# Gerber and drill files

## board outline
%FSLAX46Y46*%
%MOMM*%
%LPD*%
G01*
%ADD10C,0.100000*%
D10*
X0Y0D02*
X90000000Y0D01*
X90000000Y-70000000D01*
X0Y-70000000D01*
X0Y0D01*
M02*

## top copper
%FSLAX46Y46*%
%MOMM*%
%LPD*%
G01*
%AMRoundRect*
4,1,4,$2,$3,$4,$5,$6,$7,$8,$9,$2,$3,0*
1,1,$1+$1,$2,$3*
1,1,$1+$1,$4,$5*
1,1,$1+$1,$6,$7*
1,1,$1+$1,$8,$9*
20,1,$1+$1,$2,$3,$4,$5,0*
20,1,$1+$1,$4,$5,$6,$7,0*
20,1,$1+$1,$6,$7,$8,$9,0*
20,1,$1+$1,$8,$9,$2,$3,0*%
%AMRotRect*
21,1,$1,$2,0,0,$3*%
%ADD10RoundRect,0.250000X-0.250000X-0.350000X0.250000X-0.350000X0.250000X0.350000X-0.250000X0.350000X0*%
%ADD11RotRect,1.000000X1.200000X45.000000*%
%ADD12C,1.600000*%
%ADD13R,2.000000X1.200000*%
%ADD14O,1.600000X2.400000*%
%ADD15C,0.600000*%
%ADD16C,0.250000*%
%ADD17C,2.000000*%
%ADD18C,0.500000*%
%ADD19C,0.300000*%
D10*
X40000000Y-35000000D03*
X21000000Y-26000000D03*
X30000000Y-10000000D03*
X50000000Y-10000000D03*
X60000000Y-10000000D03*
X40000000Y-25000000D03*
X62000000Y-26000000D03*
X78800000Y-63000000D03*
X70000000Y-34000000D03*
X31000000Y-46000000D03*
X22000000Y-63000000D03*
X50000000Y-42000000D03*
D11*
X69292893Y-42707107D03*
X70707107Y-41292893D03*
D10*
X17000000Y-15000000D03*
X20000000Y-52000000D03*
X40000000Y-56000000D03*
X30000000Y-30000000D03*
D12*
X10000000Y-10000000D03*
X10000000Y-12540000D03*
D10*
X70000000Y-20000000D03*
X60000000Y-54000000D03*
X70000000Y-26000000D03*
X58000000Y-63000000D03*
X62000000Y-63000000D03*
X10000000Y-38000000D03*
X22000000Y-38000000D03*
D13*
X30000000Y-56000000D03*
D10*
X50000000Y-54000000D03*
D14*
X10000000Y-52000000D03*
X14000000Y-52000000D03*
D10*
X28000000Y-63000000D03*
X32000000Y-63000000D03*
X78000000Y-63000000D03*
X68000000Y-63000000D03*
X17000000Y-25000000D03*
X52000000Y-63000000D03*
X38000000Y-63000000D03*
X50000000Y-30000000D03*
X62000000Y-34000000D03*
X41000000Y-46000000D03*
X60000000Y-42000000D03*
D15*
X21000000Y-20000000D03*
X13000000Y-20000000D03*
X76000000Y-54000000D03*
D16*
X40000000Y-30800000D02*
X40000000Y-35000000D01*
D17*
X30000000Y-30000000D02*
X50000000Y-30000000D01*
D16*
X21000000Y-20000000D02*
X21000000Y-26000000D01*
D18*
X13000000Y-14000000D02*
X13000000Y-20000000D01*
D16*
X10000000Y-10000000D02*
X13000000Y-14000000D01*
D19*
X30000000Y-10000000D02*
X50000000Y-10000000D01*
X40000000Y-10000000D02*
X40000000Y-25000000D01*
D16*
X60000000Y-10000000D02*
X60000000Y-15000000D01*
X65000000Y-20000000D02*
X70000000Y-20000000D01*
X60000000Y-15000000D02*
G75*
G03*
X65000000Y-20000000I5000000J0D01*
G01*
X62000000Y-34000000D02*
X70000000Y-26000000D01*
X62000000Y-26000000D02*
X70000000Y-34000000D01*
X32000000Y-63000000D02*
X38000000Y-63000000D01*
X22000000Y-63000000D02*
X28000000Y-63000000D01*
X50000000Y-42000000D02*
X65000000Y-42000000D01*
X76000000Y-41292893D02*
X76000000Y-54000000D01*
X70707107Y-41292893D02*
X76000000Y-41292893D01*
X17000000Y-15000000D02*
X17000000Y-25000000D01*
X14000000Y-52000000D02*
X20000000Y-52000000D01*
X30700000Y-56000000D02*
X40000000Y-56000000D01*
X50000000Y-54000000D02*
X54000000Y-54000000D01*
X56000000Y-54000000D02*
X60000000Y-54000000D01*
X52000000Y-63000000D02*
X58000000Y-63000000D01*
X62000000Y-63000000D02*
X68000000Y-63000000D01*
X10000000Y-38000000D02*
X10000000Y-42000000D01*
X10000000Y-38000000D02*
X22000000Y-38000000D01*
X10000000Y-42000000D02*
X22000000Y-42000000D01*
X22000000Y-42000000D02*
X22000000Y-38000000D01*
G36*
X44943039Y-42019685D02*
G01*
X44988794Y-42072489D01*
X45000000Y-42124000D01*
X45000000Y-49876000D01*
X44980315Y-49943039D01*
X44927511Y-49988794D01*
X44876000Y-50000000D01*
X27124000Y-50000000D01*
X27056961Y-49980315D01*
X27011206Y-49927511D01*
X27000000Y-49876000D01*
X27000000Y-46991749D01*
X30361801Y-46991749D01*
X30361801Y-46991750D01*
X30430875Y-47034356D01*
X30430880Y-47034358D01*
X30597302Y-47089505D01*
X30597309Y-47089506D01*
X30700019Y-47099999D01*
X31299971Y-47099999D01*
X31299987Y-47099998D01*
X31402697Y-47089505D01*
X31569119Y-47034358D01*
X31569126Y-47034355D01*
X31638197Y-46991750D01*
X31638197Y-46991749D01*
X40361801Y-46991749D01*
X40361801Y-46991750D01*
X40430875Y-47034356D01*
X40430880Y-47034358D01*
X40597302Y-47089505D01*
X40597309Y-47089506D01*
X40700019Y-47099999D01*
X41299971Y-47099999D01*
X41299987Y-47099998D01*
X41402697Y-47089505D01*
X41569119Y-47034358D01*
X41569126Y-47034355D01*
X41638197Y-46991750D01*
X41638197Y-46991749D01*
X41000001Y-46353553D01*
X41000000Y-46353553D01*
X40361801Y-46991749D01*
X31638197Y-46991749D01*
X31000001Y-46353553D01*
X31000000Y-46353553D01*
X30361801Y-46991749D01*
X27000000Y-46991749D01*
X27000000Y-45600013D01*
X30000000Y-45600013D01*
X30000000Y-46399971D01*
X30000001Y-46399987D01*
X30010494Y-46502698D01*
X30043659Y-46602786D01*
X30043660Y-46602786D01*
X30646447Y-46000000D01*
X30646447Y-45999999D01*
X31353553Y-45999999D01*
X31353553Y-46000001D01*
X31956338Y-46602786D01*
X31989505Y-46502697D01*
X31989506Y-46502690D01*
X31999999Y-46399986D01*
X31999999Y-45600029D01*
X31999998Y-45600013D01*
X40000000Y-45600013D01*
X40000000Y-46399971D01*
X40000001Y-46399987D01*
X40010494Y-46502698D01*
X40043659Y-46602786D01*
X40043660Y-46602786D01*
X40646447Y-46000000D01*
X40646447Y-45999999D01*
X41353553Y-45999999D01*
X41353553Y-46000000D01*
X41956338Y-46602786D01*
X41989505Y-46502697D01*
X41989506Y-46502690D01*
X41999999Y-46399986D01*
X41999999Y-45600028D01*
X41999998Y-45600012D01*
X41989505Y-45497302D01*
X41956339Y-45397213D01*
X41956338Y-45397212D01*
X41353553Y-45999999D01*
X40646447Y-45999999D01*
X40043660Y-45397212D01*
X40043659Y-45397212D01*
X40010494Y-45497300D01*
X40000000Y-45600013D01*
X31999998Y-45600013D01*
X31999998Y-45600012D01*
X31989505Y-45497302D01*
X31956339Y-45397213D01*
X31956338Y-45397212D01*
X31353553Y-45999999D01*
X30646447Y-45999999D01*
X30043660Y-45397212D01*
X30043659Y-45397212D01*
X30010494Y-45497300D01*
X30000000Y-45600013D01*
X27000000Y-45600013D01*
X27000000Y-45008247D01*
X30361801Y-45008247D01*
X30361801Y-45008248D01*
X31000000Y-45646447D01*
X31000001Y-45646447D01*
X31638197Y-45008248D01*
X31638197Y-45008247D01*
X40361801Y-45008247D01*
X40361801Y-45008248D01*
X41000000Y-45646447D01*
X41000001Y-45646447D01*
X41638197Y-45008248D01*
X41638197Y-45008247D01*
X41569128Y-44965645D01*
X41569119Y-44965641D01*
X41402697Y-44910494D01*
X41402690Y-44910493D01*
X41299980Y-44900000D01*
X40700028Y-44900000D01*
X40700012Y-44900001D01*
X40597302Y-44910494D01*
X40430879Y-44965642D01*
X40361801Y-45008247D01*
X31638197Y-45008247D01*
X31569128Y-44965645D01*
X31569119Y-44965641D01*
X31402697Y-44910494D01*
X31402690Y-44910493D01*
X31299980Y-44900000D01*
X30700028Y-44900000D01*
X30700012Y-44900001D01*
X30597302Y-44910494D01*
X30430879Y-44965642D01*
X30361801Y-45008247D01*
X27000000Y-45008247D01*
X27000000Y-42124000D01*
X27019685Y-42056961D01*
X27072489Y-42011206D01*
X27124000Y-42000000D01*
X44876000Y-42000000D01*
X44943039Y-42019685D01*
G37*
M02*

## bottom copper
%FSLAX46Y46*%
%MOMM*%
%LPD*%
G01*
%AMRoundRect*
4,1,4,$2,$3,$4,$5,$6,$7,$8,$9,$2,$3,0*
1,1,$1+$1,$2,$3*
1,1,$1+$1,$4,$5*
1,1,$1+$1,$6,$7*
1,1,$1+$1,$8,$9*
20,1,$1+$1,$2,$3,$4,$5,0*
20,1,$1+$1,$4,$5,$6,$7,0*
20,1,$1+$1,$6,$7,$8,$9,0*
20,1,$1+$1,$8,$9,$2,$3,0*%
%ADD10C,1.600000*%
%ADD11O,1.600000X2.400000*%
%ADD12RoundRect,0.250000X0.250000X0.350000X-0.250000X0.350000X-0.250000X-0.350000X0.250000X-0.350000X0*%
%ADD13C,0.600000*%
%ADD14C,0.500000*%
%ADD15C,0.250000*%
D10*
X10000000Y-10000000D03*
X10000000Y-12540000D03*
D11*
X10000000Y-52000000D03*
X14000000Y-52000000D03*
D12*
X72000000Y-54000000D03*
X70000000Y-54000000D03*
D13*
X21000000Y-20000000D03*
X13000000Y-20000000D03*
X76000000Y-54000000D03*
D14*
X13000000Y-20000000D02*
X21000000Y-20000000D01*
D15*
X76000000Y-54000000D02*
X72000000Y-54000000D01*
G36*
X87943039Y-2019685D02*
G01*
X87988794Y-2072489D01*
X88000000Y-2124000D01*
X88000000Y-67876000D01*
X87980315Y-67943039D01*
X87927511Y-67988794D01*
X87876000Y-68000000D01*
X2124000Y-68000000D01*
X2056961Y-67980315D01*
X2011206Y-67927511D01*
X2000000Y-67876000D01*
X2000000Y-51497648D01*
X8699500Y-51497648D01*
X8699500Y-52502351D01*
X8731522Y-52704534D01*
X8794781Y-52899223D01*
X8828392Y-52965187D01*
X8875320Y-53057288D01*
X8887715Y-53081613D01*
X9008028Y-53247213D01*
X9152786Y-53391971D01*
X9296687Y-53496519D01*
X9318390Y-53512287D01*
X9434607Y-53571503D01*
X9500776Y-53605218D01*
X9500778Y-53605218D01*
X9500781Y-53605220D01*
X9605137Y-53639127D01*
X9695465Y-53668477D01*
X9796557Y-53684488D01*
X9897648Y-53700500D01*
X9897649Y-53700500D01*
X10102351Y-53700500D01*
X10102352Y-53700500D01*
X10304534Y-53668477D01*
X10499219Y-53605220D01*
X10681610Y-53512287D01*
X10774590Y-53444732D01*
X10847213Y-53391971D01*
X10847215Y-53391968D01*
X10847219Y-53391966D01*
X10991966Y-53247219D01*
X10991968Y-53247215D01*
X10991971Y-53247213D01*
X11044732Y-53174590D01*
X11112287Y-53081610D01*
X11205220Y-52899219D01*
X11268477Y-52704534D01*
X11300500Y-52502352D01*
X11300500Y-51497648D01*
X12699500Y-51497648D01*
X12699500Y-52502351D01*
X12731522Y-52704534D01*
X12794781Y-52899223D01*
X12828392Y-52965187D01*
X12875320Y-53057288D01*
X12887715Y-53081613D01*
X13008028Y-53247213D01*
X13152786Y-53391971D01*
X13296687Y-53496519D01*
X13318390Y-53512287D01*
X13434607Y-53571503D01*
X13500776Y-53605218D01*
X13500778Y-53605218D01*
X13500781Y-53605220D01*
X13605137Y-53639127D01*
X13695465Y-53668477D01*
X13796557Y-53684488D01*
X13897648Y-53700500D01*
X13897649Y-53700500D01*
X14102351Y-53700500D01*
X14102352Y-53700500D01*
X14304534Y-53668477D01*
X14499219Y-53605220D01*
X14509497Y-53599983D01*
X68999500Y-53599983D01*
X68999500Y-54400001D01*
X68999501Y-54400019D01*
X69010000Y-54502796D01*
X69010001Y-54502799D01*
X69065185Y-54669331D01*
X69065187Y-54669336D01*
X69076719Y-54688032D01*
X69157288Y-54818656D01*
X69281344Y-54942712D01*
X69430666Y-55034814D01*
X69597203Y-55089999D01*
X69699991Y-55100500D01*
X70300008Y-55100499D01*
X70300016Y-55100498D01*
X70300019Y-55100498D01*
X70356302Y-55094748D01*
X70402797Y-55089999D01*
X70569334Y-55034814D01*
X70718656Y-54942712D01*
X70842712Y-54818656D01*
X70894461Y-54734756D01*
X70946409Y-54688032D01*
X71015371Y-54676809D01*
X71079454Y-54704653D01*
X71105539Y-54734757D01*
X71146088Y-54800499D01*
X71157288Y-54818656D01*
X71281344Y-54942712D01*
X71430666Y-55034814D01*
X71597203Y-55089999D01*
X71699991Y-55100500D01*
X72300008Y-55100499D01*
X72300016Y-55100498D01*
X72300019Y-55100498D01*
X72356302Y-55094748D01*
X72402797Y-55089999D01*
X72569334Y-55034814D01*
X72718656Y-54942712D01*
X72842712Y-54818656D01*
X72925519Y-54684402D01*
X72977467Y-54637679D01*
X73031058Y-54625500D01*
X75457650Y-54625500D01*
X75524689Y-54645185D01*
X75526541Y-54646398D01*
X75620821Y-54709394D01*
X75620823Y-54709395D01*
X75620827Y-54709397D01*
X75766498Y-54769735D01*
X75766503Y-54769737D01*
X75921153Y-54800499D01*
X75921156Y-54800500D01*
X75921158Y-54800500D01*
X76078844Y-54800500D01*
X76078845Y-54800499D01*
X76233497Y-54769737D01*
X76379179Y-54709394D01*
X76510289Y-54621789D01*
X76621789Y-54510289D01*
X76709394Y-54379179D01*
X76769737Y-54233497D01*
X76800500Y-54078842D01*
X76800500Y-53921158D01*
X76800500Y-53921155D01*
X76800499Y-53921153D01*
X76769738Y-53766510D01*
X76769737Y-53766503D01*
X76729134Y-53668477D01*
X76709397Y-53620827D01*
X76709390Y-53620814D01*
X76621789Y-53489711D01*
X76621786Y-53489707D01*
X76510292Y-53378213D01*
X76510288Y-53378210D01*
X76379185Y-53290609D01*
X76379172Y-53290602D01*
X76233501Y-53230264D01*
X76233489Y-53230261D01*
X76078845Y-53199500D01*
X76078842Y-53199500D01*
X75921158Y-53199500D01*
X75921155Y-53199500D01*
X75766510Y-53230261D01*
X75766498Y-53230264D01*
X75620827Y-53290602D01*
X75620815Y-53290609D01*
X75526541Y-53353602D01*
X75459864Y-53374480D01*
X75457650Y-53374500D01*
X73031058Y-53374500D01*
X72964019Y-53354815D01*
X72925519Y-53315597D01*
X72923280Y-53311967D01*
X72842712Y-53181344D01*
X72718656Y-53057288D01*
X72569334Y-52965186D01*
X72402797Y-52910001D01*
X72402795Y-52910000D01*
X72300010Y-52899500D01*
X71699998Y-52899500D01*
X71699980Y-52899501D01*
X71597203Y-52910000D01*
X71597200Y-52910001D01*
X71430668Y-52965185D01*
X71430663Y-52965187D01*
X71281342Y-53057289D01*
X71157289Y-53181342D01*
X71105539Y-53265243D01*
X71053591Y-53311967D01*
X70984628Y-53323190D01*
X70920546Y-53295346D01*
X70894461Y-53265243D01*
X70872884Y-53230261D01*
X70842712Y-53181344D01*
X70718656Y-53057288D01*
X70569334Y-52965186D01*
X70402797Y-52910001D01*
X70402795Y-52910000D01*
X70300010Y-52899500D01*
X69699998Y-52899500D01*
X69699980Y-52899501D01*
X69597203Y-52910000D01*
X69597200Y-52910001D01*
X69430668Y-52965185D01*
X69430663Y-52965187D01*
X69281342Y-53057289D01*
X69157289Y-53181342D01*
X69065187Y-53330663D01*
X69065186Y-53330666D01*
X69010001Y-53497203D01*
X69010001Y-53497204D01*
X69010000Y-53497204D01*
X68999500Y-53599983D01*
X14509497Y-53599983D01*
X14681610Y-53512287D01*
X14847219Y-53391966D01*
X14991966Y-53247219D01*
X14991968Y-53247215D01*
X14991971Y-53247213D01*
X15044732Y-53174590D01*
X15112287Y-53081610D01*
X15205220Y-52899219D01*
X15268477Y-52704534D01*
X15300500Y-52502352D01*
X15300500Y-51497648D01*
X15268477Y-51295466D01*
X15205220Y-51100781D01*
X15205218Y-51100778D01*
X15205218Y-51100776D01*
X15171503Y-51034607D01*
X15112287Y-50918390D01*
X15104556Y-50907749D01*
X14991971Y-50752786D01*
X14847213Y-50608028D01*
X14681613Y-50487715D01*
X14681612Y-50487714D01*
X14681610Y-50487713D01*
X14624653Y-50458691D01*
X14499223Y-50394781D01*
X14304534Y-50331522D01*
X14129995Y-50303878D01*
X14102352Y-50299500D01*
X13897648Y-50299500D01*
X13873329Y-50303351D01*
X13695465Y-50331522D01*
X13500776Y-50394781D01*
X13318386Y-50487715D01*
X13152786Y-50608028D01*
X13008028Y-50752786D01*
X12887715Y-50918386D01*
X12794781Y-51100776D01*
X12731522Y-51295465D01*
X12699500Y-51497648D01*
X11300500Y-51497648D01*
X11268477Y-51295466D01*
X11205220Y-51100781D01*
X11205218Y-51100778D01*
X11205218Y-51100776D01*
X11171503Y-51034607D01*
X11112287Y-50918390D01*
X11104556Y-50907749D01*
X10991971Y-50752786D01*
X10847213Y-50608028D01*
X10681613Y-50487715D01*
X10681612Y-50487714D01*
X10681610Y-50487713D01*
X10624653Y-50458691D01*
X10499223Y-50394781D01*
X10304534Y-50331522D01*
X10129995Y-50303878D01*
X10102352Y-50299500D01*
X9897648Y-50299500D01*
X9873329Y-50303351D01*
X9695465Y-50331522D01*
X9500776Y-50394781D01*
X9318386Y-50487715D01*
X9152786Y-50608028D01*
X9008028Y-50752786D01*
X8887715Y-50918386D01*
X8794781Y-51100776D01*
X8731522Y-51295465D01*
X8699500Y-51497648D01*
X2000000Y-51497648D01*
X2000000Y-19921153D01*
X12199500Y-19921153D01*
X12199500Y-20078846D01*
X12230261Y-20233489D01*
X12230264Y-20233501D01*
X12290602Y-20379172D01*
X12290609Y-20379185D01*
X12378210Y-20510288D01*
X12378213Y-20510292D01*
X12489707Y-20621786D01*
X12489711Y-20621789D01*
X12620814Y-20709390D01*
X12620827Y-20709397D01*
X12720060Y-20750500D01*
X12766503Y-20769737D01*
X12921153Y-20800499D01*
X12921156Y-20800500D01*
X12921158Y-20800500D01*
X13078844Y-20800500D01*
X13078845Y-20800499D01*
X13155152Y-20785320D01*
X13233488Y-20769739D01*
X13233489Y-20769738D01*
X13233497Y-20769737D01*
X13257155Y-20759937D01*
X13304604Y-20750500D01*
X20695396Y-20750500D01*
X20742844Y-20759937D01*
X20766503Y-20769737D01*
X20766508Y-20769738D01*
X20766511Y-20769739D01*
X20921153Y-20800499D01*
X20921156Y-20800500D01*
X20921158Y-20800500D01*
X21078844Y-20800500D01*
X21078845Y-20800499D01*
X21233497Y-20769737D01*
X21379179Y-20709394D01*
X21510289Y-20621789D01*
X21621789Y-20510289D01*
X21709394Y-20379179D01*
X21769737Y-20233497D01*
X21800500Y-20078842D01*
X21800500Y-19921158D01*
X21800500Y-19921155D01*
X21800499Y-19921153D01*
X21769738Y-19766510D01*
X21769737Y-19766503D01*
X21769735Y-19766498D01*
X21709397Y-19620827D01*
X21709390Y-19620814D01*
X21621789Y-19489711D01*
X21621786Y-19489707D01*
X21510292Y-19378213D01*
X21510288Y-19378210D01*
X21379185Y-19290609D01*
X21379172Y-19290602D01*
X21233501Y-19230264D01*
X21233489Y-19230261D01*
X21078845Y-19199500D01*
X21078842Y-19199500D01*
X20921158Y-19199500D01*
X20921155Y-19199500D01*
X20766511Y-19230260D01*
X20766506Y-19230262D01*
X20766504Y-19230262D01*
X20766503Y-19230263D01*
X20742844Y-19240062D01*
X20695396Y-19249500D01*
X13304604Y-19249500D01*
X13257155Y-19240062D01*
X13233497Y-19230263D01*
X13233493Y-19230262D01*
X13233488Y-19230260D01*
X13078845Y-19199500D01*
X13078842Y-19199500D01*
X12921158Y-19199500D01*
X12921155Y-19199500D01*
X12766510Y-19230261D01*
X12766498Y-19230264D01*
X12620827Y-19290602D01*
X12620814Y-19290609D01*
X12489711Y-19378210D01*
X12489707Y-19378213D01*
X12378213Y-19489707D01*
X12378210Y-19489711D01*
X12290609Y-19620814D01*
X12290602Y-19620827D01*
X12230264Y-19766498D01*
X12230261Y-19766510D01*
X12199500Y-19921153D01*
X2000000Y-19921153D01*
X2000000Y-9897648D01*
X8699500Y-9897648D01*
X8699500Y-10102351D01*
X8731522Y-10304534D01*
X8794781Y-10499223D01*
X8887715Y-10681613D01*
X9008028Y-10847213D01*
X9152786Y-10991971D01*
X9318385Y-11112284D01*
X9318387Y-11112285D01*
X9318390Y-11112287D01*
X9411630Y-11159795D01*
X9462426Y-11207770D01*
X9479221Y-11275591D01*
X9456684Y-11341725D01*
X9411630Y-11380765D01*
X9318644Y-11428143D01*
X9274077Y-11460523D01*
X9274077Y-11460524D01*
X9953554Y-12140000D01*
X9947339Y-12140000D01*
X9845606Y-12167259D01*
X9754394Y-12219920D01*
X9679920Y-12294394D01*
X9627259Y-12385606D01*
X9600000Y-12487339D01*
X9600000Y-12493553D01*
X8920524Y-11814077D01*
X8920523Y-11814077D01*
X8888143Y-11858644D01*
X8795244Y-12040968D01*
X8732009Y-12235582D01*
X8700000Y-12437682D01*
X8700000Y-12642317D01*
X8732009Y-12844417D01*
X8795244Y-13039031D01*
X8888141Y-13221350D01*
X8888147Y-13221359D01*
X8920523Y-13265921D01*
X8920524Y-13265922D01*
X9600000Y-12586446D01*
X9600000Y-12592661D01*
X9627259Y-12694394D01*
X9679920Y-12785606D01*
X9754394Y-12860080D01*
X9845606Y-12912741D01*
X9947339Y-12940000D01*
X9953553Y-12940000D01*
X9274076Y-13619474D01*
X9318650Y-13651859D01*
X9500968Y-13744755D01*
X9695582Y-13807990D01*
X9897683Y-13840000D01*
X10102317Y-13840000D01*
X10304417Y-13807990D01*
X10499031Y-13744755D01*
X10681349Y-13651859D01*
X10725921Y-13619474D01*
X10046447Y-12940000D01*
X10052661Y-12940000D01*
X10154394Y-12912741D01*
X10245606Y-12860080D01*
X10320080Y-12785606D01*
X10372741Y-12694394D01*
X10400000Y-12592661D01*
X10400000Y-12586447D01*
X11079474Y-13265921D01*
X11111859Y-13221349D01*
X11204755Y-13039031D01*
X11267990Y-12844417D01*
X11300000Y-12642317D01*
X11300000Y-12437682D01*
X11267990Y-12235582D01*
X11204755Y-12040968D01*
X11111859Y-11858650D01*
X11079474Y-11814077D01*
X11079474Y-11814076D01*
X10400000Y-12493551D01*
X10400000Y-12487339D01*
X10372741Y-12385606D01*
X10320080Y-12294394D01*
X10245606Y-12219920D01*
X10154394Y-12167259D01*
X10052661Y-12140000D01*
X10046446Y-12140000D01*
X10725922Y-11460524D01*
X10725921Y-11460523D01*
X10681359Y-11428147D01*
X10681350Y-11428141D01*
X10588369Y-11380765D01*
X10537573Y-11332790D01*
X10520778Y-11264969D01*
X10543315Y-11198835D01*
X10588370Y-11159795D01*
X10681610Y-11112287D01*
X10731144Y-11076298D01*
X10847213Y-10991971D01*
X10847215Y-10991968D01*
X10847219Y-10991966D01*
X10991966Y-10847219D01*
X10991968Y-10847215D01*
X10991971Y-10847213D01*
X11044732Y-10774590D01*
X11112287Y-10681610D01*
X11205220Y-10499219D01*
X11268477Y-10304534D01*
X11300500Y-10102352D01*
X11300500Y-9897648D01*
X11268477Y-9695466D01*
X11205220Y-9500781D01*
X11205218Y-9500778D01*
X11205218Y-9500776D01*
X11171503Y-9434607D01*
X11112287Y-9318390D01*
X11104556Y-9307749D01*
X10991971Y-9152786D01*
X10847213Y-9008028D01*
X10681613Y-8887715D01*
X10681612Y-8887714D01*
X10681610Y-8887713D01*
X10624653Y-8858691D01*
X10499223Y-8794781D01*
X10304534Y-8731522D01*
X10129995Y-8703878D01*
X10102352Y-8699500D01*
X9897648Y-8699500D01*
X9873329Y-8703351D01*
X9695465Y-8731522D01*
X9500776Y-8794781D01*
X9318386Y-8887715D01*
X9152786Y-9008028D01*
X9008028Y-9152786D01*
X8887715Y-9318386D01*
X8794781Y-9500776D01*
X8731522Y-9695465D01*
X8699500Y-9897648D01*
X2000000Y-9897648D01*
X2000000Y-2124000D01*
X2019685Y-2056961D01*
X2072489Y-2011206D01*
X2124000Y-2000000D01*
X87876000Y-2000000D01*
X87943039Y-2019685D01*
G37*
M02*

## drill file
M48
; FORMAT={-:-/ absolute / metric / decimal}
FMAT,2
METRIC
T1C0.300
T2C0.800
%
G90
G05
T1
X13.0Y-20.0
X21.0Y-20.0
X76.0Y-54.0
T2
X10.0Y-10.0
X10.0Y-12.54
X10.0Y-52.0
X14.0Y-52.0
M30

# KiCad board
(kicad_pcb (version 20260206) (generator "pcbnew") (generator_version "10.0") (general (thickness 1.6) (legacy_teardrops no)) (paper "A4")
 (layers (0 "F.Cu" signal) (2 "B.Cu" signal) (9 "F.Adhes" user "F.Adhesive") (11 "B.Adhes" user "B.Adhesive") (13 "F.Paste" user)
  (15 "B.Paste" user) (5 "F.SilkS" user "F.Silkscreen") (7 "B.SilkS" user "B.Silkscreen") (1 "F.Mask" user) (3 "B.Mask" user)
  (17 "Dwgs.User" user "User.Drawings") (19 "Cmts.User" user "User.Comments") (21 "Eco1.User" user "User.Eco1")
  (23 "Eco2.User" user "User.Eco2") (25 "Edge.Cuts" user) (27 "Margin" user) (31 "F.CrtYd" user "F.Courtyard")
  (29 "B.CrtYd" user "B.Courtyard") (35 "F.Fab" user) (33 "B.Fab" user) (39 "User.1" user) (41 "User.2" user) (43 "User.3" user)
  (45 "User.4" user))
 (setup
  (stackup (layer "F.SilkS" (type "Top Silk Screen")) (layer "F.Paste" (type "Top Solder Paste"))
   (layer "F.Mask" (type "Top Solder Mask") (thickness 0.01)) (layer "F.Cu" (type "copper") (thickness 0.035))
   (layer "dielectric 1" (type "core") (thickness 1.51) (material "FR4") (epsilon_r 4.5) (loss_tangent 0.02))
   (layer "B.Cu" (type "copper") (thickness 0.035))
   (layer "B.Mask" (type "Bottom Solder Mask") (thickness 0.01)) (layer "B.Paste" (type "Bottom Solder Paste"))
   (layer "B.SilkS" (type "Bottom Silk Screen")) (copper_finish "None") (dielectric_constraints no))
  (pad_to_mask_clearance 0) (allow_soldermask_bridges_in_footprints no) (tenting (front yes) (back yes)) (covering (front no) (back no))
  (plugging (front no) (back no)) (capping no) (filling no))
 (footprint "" (layer "F.Cu") (at 40 35)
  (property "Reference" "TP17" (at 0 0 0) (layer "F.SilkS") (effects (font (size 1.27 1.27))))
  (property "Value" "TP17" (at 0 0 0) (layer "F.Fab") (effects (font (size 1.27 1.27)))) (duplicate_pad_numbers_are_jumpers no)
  (pad "1" smd roundrect (at 0 0) (size 1 1.2) (layers "F.Cu" "F.Mask" "F.Paste") (roundrect_rratio 0.25) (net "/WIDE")
   (thermal_bridge_angle 45)))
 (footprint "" (layer "F.Cu") (at 21 26)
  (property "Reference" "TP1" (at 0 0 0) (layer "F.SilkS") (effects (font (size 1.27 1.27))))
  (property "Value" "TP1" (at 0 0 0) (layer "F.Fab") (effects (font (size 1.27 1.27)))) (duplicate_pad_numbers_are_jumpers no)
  (pad "1" smd roundrect (at 0 0) (size 1 1.2) (layers "F.Cu" "F.Mask" "F.Paste") (roundrect_rratio 0.25) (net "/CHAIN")
   (thermal_bridge_angle 45)))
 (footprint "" (layer "F.Cu") (at 30 10)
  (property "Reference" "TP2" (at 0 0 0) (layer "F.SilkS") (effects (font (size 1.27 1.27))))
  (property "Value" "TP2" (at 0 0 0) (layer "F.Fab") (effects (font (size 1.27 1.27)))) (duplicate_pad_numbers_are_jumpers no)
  (pad "1" smd roundrect (at 0 0) (size 1 1.2) (layers "F.Cu" "F.Mask" "F.Paste") (roundrect_rratio 0.25) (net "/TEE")
   (thermal_bridge_angle 45)))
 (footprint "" (layer "F.Cu") (at 50 10)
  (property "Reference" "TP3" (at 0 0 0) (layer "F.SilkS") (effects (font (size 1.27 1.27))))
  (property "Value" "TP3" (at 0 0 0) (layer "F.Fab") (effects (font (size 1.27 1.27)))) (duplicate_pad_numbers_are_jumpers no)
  (pad "1" smd roundrect (at 0 0) (size 1 1.2) (layers "F.Cu" "F.Mask" "F.Paste") (roundrect_rratio 0.25) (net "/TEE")
   (thermal_bridge_angle 45)))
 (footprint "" (layer "F.Cu") (at 60 10)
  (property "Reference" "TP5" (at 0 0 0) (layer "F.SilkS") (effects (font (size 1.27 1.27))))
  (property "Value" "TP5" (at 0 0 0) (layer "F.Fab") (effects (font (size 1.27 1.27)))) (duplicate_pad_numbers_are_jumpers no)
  (pad "1" smd roundrect (at 0 0) (size 1 1.2) (layers "F.Cu" "F.Mask" "F.Paste") (roundrect_rratio 0.25) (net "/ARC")
   (thermal_bridge_angle 45)))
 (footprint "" (layer "F.Cu") (at 40 25)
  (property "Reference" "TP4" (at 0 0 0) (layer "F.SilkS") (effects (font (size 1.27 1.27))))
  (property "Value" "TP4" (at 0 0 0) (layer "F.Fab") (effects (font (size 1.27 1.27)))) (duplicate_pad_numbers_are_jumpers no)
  (pad "1" smd roundrect (at 0 0) (size 1 1.2) (layers "F.Cu" "F.Mask" "F.Paste") (roundrect_rratio 0.25) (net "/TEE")
   (thermal_bridge_angle 45)))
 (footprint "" (layer "F.Cu") (at 62 26)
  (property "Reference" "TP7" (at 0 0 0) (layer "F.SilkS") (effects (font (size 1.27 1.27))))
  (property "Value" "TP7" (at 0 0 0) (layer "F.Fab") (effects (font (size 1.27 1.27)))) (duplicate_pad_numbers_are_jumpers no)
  (pad "1" smd roundrect (at 0 0) (size 1 1.2) (layers "F.Cu" "F.Mask" "F.Paste") (roundrect_rratio 0.25) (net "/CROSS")
   (thermal_bridge_angle 45)))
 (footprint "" (layer "F.Cu") (at 78.8 63)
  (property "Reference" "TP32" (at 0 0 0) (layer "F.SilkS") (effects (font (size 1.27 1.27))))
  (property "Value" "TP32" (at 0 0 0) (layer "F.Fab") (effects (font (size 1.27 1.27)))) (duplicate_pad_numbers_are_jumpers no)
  (pad "1" smd roundrect (at 0 0) (size 1 1.2) (layers "F.Cu" "F.Mask" "F.Paste") (roundrect_rratio 0.25) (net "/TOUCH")
   (thermal_bridge_angle 45)))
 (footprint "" (layer "F.Cu") (at 70 34)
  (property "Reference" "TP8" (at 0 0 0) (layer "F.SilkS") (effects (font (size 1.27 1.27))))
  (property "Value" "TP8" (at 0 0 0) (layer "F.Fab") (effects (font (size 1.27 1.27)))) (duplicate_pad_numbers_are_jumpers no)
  (pad "1" smd roundrect (at 0 0) (size 1 1.2) (layers "F.Cu" "F.Mask" "F.Paste") (roundrect_rratio 0.25) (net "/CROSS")
   (thermal_bridge_angle 45)))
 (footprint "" (layer "F.Cu") (at 31 46)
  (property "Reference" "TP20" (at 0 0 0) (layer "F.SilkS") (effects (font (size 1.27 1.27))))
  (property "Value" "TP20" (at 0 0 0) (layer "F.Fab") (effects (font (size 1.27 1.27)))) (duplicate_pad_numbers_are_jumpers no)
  (pad "1" smd roundrect (at 0 0) (size 1 1.2) (layers "F.Cu" "F.Mask" "F.Paste") (roundrect_rratio 0.25) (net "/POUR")
   (thermal_bridge_angle 45)))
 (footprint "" (layer "F.Cu") (at 22 63)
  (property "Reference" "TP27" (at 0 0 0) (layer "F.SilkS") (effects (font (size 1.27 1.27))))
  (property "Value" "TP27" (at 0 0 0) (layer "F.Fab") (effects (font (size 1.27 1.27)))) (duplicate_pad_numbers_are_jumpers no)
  (pad "1" smd roundrect (at 0 0) (size 1 1.2) (layers "F.Cu" "F.Mask" "F.Paste") (roundrect_rratio 0.25) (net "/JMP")
   (thermal_bridge_angle 45)))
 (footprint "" (layer "F.Cu") (at 50 42)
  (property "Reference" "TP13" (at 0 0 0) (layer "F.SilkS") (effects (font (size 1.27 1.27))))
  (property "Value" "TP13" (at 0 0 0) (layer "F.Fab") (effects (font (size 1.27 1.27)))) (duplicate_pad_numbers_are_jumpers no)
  (pad "1" smd roundrect (at 0 0) (size 1 1.2) (layers "F.Cu" "F.Mask" "F.Paste") (roundrect_rratio 0.25) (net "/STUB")
   (thermal_bridge_angle 45)))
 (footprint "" (layer "F.Cu") (at 70 42 45)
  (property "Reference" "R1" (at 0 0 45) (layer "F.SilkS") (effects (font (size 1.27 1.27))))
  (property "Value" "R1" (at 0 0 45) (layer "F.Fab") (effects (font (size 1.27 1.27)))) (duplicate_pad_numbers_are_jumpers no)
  (pad "1" smd rect (at -1 0 45) (size 1 1.2) (layers "F.Cu" "F.Mask" "F.Paste") (thermal_bridge_angle 45))
  (pad "2" smd rect (at 1 0 45) (size 1 1.2) (layers "F.Cu" "F.Mask" "F.Paste") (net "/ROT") (thermal_bridge_angle 45)))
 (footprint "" (layer "F.Cu") (at 17 15)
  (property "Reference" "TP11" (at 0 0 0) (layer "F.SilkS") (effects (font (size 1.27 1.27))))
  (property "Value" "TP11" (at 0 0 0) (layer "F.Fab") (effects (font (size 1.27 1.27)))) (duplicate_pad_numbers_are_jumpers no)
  (pad "1" smd roundrect (at 0 0) (size 1 1.2) (layers "F.Cu" "F.Mask" "F.Paste") (roundrect_rratio 0.25) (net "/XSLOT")
   (thermal_bridge_angle 45)))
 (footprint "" (layer "F.Cu") (at 20 52)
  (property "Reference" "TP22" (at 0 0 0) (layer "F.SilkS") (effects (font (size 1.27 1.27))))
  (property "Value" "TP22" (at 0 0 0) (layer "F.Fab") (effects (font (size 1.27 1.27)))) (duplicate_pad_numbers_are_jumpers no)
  (pad "1" smd roundrect (at 0 0) (size 1 1.2) (layers "F.Cu" "F.Mask" "F.Paste") (roundrect_rratio 0.25) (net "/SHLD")
   (thermal_bridge_angle 45)))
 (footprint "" (layer "F.Cu") (at 40 56)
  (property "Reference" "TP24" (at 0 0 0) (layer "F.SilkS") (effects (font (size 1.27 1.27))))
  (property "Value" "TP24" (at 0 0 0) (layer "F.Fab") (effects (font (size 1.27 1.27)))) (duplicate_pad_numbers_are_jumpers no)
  (pad "1" smd roundrect (at 0 0) (size 1 1.2) (layers "F.Cu" "F.Mask" "F.Paste") (roundrect_rratio 0.25) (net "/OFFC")
   (thermal_bridge_angle 45)))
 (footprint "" (layer "F.Cu") (at 30 30)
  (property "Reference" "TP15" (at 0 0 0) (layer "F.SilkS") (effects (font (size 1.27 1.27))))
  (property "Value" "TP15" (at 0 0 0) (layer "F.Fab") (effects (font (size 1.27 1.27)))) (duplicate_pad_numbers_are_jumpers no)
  (pad "1" smd roundrect (at 0 0) (size 1 1.2) (layers "F.Cu" "F.Mask" "F.Paste") (roundrect_rratio 0.25) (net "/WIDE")
   (thermal_bridge_angle 45)))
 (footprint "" (layer "F.Cu") (at 10 10)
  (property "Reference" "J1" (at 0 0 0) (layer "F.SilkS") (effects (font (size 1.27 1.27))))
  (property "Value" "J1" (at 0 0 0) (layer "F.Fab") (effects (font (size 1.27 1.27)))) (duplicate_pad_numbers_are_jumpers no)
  (pad "1" thru_hole circle (at 0 0) (size 1.6 1.6) (drill 0.8) (layers "*.Cu" "*.Mask") (remove_unused_layers no) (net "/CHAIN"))
  (pad "2" thru_hole circle (at 0 2.54) (size 1.6 1.6) (drill 0.8) (layers "*.Cu" "*.Mask") (remove_unused_layers no) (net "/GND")))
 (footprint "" (layer "F.Cu") (at 70 20)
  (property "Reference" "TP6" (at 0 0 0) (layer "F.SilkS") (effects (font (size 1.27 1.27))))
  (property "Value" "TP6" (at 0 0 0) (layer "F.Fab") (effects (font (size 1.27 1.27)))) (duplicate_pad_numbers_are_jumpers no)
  (pad "1" smd roundrect (at 0 0) (size 1 1.2) (layers "F.Cu" "F.Mask" "F.Paste") (roundrect_rratio 0.25) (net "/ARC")
   (thermal_bridge_angle 45)))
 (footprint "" (layer "F.Cu") (at 60 54)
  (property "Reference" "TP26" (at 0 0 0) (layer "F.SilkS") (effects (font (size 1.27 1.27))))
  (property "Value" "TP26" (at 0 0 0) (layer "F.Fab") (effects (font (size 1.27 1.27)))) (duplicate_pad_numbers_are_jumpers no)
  (pad "1" smd roundrect (at 0 0) (size 1 1.2) (layers "F.Cu" "F.Mask" "F.Paste") (roundrect_rratio 0.25) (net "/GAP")
   (thermal_bridge_angle 45)))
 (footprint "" (layer "F.Cu") (at 70 26)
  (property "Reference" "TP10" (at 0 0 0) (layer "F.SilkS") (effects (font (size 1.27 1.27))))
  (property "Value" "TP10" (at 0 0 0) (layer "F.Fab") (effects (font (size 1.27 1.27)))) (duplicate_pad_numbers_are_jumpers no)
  (pad "1" smd roundrect (at 0 0) (size 1 1.2) (layers "F.Cu" "F.Mask" "F.Paste") (roundrect_rratio 0.25) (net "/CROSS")
   (thermal_bridge_angle 45)))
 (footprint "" (layer "F.Cu") (at 60 63)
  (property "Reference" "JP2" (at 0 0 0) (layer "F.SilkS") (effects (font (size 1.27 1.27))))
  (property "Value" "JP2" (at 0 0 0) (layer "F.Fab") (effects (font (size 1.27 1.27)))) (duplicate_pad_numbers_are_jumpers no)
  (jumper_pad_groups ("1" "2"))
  (pad "1" smd roundrect (at -2 0) (size 1 1.2) (layers "F.Cu" "F.Mask" "F.Paste") (roundrect_rratio 0.25) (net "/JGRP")
   (thermal_bridge_angle 45))
  (pad "2" smd roundrect (at 2 0) (size 1 1.2) (layers "F.Cu" "F.Mask" "F.Paste") (roundrect_rratio 0.25) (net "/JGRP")
   (thermal_bridge_angle 45)))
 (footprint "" (layer "F.Cu") (at 10 38)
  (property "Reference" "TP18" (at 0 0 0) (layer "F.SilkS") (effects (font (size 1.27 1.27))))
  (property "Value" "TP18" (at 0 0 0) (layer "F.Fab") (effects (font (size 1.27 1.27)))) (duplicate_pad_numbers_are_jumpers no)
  (pad "1" smd roundrect (at 0 0) (size 1 1.2) (layers "F.Cu" "F.Mask" "F.Paste") (roundrect_rratio 0.25) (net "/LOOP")
   (thermal_bridge_angle 45)))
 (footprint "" (layer "F.Cu") (at 22 38)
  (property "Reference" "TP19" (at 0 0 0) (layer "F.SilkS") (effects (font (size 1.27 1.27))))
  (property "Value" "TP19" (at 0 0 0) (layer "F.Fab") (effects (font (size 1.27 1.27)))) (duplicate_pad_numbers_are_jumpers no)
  (pad "1" smd roundrect (at 0 0) (size 1 1.2) (layers "F.Cu" "F.Mask" "F.Paste") (roundrect_rratio 0.25) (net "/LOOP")
   (thermal_bridge_angle 45)))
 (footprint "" (layer "F.Cu") (at 30 56)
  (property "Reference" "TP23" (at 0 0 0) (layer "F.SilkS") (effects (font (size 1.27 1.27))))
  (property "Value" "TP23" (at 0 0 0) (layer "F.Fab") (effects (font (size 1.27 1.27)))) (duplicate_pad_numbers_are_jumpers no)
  (pad "1" smd rect (at 0 0) (size 2 1.2) (layers "F.Cu" "F.Mask" "F.Paste") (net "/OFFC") (thermal_bridge_angle 45)))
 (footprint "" (layer "F.Cu") (at 50 54)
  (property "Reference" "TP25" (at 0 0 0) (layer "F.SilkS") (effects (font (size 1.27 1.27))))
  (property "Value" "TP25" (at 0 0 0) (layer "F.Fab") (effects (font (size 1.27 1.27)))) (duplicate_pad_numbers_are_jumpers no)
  (pad "1" smd roundrect (at 0 0) (size 1 1.2) (layers "F.Cu" "F.Mask" "F.Paste") (roundrect_rratio 0.25) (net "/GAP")
   (thermal_bridge_angle 45)))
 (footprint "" (layer "F.Cu") (at 12 52)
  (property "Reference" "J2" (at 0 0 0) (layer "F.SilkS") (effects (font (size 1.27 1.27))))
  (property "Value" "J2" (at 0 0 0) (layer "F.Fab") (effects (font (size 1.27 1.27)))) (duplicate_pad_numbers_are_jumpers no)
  (pad "S" thru_hole oval (at -2 0) (size 1.6 2.4) (drill 0.8) (layers "*.Cu" "*.Mask") (remove_unused_layers no) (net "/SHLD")
   (thermal_bridge_angle 45))
  (pad "S" thru_hole oval (at 2 0) (size 1.6 2.4) (drill 0.8) (layers "*.Cu" "*.Mask") (remove_unused_layers no) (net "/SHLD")
   (thermal_bridge_angle 45)))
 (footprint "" (layer "F.Cu") (at 30 63)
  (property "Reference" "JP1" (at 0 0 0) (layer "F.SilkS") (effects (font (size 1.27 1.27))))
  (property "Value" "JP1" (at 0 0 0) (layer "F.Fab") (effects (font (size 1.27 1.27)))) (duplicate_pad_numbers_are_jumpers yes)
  (pad "1" smd roundrect (at -2 0) (size 1 1.2) (layers "F.Cu" "F.Mask" "F.Paste") (roundrect_rratio 0.25) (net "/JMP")
   (thermal_bridge_angle 45))
  (pad "1" smd roundrect (at 2 0) (size 1 1.2) (layers "F.Cu" "F.Mask" "F.Paste") (roundrect_rratio 0.25) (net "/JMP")
   (thermal_bridge_angle 45)))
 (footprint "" (layer "F.Cu") (at 78 63)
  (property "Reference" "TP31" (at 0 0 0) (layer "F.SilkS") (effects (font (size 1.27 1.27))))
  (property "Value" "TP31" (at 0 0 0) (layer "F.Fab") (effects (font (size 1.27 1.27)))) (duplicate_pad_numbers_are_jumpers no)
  (pad "1" smd roundrect (at 0 0) (size 1 1.2) (layers "F.Cu" "F.Mask" "F.Paste") (roundrect_rratio 0.25) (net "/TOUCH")
   (thermal_bridge_angle 45)))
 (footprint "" (layer "F.Cu") (at 68 63)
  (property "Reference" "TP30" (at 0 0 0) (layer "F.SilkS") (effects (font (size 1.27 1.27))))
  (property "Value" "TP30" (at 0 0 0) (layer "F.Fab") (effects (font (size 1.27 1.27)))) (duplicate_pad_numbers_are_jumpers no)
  (pad "1" smd roundrect (at 0 0) (size 1 1.2) (layers "F.Cu" "F.Mask" "F.Paste") (roundrect_rratio 0.25) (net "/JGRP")
   (thermal_bridge_angle 45)))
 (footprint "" (layer "F.Cu") (at 17 25)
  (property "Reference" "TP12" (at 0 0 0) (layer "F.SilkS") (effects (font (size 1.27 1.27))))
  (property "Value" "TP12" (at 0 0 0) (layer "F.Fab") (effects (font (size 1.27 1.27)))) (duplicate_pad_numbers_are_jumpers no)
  (pad "1" smd roundrect (at 0 0) (size 1 1.2) (layers "F.Cu" "F.Mask" "F.Paste") (roundrect_rratio 0.25) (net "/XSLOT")
   (thermal_bridge_angle 45)))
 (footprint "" (layer "F.Cu") (at 52 63)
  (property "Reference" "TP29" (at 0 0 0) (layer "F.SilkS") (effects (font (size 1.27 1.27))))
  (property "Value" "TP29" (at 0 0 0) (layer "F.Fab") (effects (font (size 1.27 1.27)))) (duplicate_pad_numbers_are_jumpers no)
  (pad "1" smd roundrect (at 0 0) (size 1 1.2) (layers "F.Cu" "F.Mask" "F.Paste") (roundrect_rratio 0.25) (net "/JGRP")
   (thermal_bridge_angle 45)))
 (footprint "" (layer "F.Cu") (at 38 63)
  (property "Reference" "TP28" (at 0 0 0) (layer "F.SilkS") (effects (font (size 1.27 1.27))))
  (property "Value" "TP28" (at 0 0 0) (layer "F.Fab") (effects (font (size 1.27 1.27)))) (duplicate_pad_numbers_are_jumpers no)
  (pad "1" smd roundrect (at 0 0) (size 1 1.2) (layers "F.Cu" "F.Mask" "F.Paste") (roundrect_rratio 0.25) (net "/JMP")
   (thermal_bridge_angle 45)))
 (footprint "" (layer "F.Cu") (at 50 30)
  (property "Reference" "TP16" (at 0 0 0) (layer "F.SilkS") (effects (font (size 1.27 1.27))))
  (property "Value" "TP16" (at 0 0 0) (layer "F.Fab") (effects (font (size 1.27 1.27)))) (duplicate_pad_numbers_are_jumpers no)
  (pad "1" smd roundrect (at 0 0) (size 1 1.2) (layers "F.Cu" "F.Mask" "F.Paste") (roundrect_rratio 0.25) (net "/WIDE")
   (thermal_bridge_angle 45)))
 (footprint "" (layer "F.Cu") (at 62 34)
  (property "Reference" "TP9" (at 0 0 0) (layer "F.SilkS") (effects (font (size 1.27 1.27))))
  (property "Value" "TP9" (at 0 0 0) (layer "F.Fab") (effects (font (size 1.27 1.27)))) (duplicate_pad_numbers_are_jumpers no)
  (pad "1" smd roundrect (at 0 0) (size 1 1.2) (layers "F.Cu" "F.Mask" "F.Paste") (roundrect_rratio 0.25) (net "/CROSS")
   (thermal_bridge_angle 45)))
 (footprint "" (layer "F.Cu") (at 41 46)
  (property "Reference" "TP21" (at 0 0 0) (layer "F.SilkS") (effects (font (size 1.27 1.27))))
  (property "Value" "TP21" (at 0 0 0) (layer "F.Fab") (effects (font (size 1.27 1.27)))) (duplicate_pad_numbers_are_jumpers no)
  (pad "1" smd roundrect (at 0 0) (size 1 1.2) (layers "F.Cu" "F.Mask" "F.Paste") (roundrect_rratio 0.25) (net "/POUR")
   (thermal_bridge_angle 45)))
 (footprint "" (layer "F.Cu") (at 60 42)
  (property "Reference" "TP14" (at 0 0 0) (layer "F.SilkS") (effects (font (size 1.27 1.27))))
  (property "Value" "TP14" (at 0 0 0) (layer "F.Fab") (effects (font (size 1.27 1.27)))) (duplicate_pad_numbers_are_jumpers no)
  (pad "1" smd roundrect (at 0 0) (size 1 1.2) (layers "F.Cu" "F.Mask" "F.Paste") (roundrect_rratio 0.25) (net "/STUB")
   (thermal_bridge_angle 45)))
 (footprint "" (layer "B.Cu") (at 71 54 180)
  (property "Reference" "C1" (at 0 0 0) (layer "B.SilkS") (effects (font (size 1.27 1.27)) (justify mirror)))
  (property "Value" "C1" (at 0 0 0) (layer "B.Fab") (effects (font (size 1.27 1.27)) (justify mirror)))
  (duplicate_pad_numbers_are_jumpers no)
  (pad "1" smd roundrect (at -1 0 180) (size 1 1.2) (layers "B.Cu" "B.Mask" "B.Paste") (roundrect_rratio 0.25) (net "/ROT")
   (thermal_bridge_angle 45))
  (pad "2" smd roundrect (at 1 0 180) (size 1 1.2) (layers "B.Cu" "B.Mask" "B.Paste") (roundrect_rratio 0.25) (thermal_bridge_angle 45)))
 (gr_rect (start 0 0) (end 90 70) (stroke (width 0.1) (type default)) (fill no) (layer "Edge.Cuts"))
 (segment (start 40 30.8) (end 40 35) (width 0.25) (layer "F.Cu") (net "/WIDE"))
 (segment (start 30 30) (end 50 30) (width 2) (layer "F.Cu") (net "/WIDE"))
 (segment (start 21 20) (end 21 26) (width 0.25) (layer "F.Cu") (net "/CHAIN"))
 (segment (start 13 14) (end 13 20) (width 0.5) (layer "F.Cu") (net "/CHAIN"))
 (segment (start 10 10) (end 13 14) (width 0.25) (layer "F.Cu") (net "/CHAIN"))
 (via (at 21 20) (size 0.6) (drill 0.3) (layers "F.Cu" "B.Cu") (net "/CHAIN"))
 (via (at 13 20) (size 0.6) (drill 0.3) (layers "F.Cu" "B.Cu") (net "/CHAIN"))
 (segment (start 13 20) (end 21 20) (width 0.5) (layer "B.Cu") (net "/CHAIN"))
 (segment (start 30 10) (end 50 10) (width 0.3) (layer "F.Cu") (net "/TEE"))
 (segment (start 40 10) (end 40 25) (width 0.3) (layer "F.Cu") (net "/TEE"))
 (segment (start 60 10) (end 60 15) (width 0.25) (layer "F.Cu") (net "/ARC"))
 (segment (start 65 20) (end 70 20) (width 0.25) (layer "F.Cu") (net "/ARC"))
 (arc (start 60 15) (mid 61.464466 18.535533) (end 65 20) (width 0.25) (layer "F.Cu") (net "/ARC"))
 (segment (start 62 34) (end 70 26) (width 0.25) (layer "F.Cu") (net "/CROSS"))
 (segment (start 62 26) (end 70 34) (width 0.25) (layer "F.Cu") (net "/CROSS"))
 (segment (start 32 63) (end 38 63) (width 0.25) (layer "F.Cu") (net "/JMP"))
 (segment (start 22 63) (end 28 63) (width 0.25) (layer "F.Cu") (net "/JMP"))
 (segment (start 50 42) (end 65 42) (width 0.25) (layer "F.Cu") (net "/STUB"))
 (segment (start 76 41.292893) (end 76 54) (width 0.25) (layer "F.Cu") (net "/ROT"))
 (segment (start 70.707107 41.292893) (end 76 41.292893) (width 0.25) (layer "F.Cu") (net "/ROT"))
 (via (at 76 54) (size 0.6) (drill 0.3) (layers "F.Cu" "B.Cu") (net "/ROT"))
 (segment (start 76 54) (end 72 54) (width 0.25) (layer "B.Cu") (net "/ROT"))
 (segment (start 17 15) (end 17 25) (width 0.25) (layer "F.Cu") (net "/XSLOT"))
 (segment (start 14 52) (end 20 52) (width 0.25) (layer "F.Cu") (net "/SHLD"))
 (segment (start 30.7 56) (end 40 56) (width 0.25) (layer "F.Cu") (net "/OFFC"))
 (segment (start 50 54) (end 54 54) (width 0.25) (layer "F.Cu") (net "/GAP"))
 (segment (start 56 54) (end 60 54) (width 0.25) (layer "F.Cu") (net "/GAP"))
 (segment (start 52 63) (end 58 63) (width 0.25) (layer "F.Cu") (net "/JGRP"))
 (segment (start 62 63) (end 68 63) (width 0.25) (layer "F.Cu") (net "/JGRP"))
 (segment (start 10 38) (end 10 42) (width 0.25) (layer "F.Cu") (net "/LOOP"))
 (segment (start 10 38) (end 22 38) (width 0.25) (layer "F.Cu") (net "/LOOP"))
 (segment (start 10 42) (end 22 42) (width 0.25) (layer "F.Cu") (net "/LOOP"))
 (segment (start 22 42) (end 22 38) (width 0.25) (layer "F.Cu") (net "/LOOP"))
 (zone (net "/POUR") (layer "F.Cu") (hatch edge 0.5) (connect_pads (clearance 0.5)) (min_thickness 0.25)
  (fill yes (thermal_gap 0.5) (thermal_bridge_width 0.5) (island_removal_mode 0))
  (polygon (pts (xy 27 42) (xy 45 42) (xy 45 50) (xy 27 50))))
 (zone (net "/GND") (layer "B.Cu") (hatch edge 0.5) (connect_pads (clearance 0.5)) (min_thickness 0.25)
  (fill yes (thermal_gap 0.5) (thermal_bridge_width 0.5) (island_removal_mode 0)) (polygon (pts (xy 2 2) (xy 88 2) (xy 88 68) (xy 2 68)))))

